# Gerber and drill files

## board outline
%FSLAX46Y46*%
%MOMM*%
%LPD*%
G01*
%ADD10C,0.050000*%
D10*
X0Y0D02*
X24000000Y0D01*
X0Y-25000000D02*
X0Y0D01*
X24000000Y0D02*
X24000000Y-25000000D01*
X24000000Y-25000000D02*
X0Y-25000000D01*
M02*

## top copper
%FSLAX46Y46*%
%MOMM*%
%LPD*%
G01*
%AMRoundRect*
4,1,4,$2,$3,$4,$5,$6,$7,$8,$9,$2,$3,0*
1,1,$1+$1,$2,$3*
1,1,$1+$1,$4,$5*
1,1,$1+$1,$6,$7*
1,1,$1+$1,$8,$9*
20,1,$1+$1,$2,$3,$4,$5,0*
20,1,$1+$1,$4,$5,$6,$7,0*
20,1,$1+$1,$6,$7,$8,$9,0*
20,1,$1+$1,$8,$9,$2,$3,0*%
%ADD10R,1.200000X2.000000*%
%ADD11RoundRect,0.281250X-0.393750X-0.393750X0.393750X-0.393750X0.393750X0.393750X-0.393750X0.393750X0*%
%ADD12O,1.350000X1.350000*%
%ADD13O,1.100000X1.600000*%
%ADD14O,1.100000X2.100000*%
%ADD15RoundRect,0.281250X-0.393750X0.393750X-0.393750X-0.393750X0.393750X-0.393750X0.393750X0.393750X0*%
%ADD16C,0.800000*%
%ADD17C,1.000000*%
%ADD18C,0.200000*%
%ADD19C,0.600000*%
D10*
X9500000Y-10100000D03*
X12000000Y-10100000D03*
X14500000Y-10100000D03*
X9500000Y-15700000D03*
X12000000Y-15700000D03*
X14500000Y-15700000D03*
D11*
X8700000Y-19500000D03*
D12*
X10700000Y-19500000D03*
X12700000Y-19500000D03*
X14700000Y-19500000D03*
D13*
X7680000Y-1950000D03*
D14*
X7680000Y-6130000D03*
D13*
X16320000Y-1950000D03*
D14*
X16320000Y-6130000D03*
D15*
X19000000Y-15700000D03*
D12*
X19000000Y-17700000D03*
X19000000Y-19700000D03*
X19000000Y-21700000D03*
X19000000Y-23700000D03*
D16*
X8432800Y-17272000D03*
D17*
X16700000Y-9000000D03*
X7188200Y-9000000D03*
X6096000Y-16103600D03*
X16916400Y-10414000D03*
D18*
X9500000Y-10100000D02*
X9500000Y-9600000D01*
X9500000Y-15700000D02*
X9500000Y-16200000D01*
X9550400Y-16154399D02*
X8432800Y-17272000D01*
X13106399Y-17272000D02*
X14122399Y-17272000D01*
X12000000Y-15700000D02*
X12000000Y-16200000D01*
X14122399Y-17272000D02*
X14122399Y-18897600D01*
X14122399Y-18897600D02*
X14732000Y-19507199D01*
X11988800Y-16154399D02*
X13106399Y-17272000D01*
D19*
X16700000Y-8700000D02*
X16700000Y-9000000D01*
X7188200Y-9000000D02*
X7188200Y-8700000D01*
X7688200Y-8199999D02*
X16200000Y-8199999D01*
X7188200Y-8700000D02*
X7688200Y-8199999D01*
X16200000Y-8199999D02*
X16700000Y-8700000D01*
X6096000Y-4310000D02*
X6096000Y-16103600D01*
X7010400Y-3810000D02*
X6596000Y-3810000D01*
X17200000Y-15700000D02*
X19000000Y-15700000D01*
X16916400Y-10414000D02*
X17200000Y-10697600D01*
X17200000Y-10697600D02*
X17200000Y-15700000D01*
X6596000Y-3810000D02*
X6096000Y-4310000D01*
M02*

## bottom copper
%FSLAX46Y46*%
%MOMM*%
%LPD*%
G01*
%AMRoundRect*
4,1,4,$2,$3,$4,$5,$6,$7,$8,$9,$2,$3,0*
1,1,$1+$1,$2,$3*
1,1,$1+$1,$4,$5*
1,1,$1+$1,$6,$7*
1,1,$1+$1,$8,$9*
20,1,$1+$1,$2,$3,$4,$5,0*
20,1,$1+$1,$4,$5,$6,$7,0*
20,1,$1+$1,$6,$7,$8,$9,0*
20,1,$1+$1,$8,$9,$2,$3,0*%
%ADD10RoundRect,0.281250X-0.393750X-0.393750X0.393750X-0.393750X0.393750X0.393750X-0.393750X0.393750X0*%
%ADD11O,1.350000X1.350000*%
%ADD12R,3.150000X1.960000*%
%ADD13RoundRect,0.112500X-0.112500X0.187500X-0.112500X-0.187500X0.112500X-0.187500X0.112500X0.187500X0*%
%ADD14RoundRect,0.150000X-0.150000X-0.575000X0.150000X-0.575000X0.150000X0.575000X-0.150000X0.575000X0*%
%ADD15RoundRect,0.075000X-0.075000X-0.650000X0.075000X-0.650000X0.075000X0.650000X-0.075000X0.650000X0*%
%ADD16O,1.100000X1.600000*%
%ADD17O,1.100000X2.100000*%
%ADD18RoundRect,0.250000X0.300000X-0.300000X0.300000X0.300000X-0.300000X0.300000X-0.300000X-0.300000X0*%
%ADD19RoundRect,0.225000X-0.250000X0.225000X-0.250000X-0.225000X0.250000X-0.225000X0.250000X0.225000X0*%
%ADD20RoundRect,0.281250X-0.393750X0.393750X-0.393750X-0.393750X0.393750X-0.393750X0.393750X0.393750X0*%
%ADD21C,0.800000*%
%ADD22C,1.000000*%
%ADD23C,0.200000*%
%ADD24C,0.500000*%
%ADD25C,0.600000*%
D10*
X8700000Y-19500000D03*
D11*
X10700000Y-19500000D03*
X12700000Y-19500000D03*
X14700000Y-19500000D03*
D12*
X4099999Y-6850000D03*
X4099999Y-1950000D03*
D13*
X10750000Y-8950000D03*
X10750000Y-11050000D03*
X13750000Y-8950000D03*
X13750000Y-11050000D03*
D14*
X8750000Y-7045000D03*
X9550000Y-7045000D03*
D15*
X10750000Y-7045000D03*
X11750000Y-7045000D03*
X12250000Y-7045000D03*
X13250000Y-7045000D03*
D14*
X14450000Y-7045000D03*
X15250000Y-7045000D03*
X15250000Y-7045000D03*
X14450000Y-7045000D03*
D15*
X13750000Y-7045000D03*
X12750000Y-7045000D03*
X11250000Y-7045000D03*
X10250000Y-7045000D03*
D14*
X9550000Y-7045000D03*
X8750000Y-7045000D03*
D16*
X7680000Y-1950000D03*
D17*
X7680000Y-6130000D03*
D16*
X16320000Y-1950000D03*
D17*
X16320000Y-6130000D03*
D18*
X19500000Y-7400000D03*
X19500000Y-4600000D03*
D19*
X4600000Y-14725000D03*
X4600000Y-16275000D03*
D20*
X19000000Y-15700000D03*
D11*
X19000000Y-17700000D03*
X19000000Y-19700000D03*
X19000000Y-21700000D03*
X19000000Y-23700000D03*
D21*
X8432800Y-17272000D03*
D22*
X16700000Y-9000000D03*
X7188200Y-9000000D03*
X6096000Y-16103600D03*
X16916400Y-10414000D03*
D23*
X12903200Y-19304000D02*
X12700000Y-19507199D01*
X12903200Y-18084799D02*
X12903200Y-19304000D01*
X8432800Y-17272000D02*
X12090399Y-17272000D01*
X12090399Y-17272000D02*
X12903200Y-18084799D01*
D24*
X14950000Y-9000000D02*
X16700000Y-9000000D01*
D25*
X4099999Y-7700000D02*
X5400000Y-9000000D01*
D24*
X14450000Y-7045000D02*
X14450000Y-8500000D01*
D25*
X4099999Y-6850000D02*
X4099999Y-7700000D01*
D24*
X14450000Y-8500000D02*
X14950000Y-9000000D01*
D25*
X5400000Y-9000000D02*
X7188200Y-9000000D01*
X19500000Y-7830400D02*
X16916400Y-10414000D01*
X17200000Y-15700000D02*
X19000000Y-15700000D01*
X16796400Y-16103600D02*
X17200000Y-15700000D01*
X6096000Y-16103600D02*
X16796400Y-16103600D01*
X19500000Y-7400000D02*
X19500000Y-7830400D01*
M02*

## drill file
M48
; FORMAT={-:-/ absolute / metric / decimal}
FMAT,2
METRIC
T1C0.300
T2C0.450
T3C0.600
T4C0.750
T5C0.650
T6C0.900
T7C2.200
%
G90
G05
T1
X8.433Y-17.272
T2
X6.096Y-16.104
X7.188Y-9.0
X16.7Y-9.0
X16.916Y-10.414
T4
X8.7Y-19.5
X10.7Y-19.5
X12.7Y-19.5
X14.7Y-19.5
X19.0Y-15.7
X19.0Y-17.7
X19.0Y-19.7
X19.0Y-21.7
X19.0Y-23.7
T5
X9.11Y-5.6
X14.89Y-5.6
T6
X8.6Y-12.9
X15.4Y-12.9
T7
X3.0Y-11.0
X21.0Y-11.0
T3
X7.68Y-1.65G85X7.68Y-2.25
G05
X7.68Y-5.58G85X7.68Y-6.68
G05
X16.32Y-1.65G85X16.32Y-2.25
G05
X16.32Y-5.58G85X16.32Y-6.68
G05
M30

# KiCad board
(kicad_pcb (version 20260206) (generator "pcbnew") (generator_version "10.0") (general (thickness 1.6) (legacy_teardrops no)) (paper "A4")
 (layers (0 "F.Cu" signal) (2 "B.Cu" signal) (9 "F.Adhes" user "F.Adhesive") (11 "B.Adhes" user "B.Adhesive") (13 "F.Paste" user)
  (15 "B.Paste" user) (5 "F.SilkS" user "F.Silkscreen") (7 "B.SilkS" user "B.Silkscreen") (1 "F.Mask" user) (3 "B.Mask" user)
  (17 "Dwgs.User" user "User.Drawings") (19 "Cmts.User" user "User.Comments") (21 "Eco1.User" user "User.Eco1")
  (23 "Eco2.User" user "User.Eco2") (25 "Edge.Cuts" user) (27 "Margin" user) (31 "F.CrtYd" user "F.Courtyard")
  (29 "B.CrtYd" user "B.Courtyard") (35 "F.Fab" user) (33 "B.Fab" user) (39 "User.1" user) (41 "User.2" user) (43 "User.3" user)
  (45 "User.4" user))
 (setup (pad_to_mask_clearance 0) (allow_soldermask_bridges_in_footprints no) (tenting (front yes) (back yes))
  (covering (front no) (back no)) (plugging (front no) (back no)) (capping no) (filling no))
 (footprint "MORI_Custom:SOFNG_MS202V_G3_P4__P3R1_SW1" (layer "F.Cu") (at 12 12.9)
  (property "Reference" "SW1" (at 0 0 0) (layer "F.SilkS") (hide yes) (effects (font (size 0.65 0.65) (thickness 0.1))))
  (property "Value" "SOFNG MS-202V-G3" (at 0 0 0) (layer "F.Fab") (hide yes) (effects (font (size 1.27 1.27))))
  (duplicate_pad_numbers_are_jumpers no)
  (pad "" np_thru_hole circle (at -3.4 0) (size 0.9 0.9) (drill 0.9) (layers "*.Cu" "*.Mask"))
  (pad "" np_thru_hole circle (at 3.4 0) (size 0.9 0.9) (drill 0.9) (layers "*.Cu" "*.Mask"))
  (pad "1" smd rect (at -2.5 -2.8) (size 1.2 2) (layers "F.Cu" "F.Mask" "F.Paste") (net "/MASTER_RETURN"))
  (pad "2" smd rect (at 0 -2.8) (size 1.2 2) (layers "F.Cu" "F.Mask" "F.Paste") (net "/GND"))
  (pad "3" smd rect (at 2.5 -2.8) (size 1.2 2) (layers "F.Cu" "F.Mask" "F.Paste") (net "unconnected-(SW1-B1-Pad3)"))
  (pad "4" smd rect (at -2.5 2.8) (size 1.2 2) (layers "F.Cu" "F.Mask" "F.Paste") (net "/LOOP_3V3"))
  (pad "5" smd rect (at 0 2.8) (size 1.2 2) (layers "F.Cu" "F.Mask" "F.Paste") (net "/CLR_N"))
  (pad "6" smd rect (at 2.5 2.8) (size 1.2 2) (layers "F.Cu" "F.Mask" "F.Paste") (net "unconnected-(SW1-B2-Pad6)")))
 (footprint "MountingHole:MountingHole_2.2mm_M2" (layer "F.Cu") (at 3 11)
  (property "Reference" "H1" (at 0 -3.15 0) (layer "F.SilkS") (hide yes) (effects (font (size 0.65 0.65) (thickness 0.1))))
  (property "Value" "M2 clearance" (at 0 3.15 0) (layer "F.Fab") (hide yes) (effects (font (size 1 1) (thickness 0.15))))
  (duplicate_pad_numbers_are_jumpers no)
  (pad "" np_thru_hole circle (at 0 0) (size 2.2 2.2) (drill 2.2) (layers "*.Cu" "*.Mask")))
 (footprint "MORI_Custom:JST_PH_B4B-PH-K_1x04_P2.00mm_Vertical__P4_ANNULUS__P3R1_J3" (layer "F.Cu") (at 8.7 19.5)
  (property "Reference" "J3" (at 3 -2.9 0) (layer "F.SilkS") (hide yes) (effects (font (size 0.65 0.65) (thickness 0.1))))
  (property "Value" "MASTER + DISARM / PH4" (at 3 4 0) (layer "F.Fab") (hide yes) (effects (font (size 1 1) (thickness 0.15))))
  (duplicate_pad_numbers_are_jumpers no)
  (pad "1" thru_hole roundrect (at 0 0) (size 1.35 1.35) (drill 0.75) (layers "*.Cu" "*.Mask") (remove_unused_layers no)
   (roundrect_rratio 0.208333) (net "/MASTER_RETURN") (thermal_bridge_width 0.299999) (thermal_bridge_angle 45) (thermal_gap 0.254))
  (pad "2" thru_hole oval (at 2 0) (size 1.35 1.35) (drill 0.75) (layers "*.Cu" "*.Mask") (remove_unused_layers no) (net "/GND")
   (thermal_bridge_width 0.299999) (thermal_bridge_angle 45) (thermal_gap 0.254))
  (pad "3" thru_hole oval (at 4 0) (size 1.35 1.35) (drill 0.75) (layers "*.Cu" "*.Mask") (remove_unused_layers no) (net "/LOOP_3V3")
   (thermal_bridge_width 0.299999) (thermal_bridge_angle 45) (thermal_gap 0.254))
  (pad "4" thru_hole oval (at 6 0) (size 1.35 1.35) (drill 0.75) (layers "*.Cu" "*.Mask") (remove_unused_layers no) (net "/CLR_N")
   (thermal_bridge_width 0.299999) (thermal_bridge_angle 45) (thermal_gap 0.254)))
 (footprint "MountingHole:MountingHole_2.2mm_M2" (layer "F.Cu") (at 21 11)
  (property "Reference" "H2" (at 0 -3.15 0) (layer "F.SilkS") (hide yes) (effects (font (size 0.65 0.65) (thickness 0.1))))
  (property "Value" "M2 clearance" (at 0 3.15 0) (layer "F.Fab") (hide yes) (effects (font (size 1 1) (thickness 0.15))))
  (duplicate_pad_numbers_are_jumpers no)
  (pad "" np_thru_hole circle (at 0 0) (size 2.2 2.2) (drill 2.2) (layers "*.Cu" "*.Mask")))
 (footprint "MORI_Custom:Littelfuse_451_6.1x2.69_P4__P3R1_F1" (layer "B.Cu") (at 4.099999 4.4 90)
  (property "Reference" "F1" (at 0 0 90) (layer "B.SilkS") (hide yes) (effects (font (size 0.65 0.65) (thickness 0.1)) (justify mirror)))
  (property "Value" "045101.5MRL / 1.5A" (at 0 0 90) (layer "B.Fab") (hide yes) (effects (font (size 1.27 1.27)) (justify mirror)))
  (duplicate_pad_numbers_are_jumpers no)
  (pad "1" smd rect (at -2.45 0 90) (size 1.96 3.15) (layers "B.Cu" "B.Mask" "B.Paste") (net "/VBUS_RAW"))
  (pad "2" smd rect (at 2.45 0 90) (size 1.96 3.15) (layers "B.Cu" "B.Mask" "B.Paste") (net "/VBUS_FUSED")))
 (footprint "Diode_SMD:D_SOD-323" (layer "B.Cu") (at 10.75 10 -90)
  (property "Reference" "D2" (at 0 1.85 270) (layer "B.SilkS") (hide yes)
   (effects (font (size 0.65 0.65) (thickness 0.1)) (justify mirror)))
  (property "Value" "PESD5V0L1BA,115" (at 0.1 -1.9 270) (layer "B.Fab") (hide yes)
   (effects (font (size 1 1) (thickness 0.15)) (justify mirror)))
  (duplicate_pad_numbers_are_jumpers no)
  (pad "1" smd roundrect (at -1.05 0 270) (size 0.6 0.45) (layers "B.Cu" "B.Mask" "B.Paste") (roundrect_rratio 0.25) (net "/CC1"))
  (pad "2" smd roundrect (at 1.05 0 270) (size 0.6 0.45) (layers "B.Cu" "B.Mask" "B.Paste") (roundrect_rratio 0.25) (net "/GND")))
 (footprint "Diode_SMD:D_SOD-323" (layer "B.Cu") (at 13.75 10 -90)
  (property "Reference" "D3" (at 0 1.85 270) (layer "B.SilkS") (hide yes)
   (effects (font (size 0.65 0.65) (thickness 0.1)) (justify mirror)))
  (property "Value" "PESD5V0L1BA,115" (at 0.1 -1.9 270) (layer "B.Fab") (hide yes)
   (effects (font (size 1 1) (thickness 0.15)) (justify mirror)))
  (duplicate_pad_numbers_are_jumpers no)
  (pad "1" smd roundrect (at -1.05 0 270) (size 0.6 0.45) (layers "B.Cu" "B.Mask" "B.Paste") (roundrect_rratio 0.25) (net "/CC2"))
  (pad "2" smd roundrect (at 1.05 0 270) (size 0.6 0.45) (layers "B.Cu" "B.Mask" "B.Paste") (roundrect_rratio 0.25) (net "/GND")))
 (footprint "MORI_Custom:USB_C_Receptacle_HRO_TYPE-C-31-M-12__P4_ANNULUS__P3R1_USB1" (layer "B.Cu") (at 12 3)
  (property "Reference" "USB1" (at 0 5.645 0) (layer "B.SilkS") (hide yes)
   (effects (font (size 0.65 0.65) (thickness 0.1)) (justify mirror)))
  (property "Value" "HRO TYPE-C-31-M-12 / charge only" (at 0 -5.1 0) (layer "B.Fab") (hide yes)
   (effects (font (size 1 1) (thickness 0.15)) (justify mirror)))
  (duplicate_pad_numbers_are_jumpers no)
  (pad "" np_thru_hole circle (at -2.89 2.6) (size 0.65 0.65) (drill 0.65) (layers "*.Cu" "*.Mask"))
  (pad "" np_thru_hole circle (at 2.89 2.6) (size 0.65 0.65) (drill 0.65) (layers "*.Cu" "*.Mask"))
  (pad "A1" smd roundrect (at -3.25 4.045) (size 0.6 1.45) (layers "B.Cu" "B.Mask" "B.Paste") (roundrect_rratio 0.25) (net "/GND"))
  (pad "A4" smd roundrect (at -2.45 4.045) (size 0.6 1.45) (layers "B.Cu" "B.Mask" "B.Paste") (roundrect_rratio 0.25) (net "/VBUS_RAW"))
  (pad "A5" smd roundrect (at -1.25 4.045) (size 0.3 1.45) (layers "B.Cu" "B.Mask" "B.Paste") (roundrect_rratio 0.25) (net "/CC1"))
  (pad "A6" smd roundrect (at -0.25 4.045) (size 0.3 1.45) (layers "B.Cu" "B.Mask" "B.Paste") (roundrect_rratio 0.25)
   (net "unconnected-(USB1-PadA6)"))
  (pad "A7" smd roundrect (at 0.25 4.045) (size 0.3 1.45) (layers "B.Cu" "B.Mask" "B.Paste") (roundrect_rratio 0.25)
   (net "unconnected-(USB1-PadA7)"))
  (pad "A8" smd roundrect (at 1.25 4.045) (size 0.3 1.45) (layers "B.Cu" "B.Mask" "B.Paste") (roundrect_rratio 0.25)
   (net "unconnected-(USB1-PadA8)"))
  (pad "A9" smd roundrect (at 2.45 4.045) (size 0.6 1.45) (layers "B.Cu" "B.Mask" "B.Paste") (roundrect_rratio 0.25) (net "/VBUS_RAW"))
  (pad "A12" smd roundrect (at 3.25 4.045) (size 0.6 1.45) (layers "B.Cu" "B.Mask" "B.Paste") (roundrect_rratio 0.25) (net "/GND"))
  (pad "B1" smd roundrect (at 3.25 4.045) (size 0.6 1.45) (layers "B.Cu" "B.Mask" "B.Paste") (roundrect_rratio 0.25) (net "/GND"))
  (pad "B4" smd roundrect (at 2.45 4.045) (size 0.6 1.45) (layers "B.Cu" "B.Mask" "B.Paste") (roundrect_rratio 0.25) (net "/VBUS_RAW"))
  (pad "B5" smd roundrect (at 1.75 4.045) (size 0.3 1.45) (layers "B.Cu" "B.Mask" "B.Paste") (roundrect_rratio 0.25) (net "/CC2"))
  (pad "B6" smd roundrect (at 0.75 4.045) (size 0.3 1.45) (layers "B.Cu" "B.Mask" "B.Paste") (roundrect_rratio 0.25)
   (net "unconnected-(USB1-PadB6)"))
  (pad "B7" smd roundrect (at -0.75 4.045) (size 0.3 1.45) (layers "B.Cu" "B.Mask" "B.Paste") (roundrect_rratio 0.25)
   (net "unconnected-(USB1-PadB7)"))
  (pad "B8" smd roundrect (at -1.75 4.045) (size 0.3 1.45) (layers "B.Cu" "B.Mask" "B.Paste") (roundrect_rratio 0.25)
   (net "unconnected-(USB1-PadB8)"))
  (pad "B9" smd roundrect (at -2.45 4.045) (size 0.6 1.45) (layers "B.Cu" "B.Mask" "B.Paste") (roundrect_rratio 0.25) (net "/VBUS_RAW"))
  (pad "B12" smd roundrect (at -3.25 4.045) (size 0.6 1.45) (layers "B.Cu" "B.Mask" "B.Paste") (roundrect_rratio 0.25) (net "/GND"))
  (pad "SH" thru_hole oval (at -4.32 -1.05) (size 1.1 1.6) (drill oval 0.6 1.2) (layers "*.Cu" "*.Mask") (remove_unused_layers no)
   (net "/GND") (thermal_bridge_width 0.299999) (thermal_bridge_angle 45) (thermal_gap 0.254))
  (pad "SH" thru_hole oval (at -4.32 3.13) (size 1.1 2.1) (drill oval 0.6 1.7) (layers "*.Cu" "*.Mask") (remove_unused_layers no)
   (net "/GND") (thermal_bridge_width 0.299999) (thermal_bridge_angle 45) (thermal_gap 0.254))
  (pad "SH" thru_hole oval (at 4.32 -1.05) (size 1.1 1.6) (drill oval 0.6 1.2) (layers "*.Cu" "*.Mask") (remove_unused_layers no)
   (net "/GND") (thermal_bridge_width 0.299999) (thermal_bridge_angle 45) (thermal_gap 0.254))
  (pad "SH" thru_hole oval (at 4.32 3.13) (size 1.1 2.1) (drill oval 0.6 1.7) (layers "*.Cu" "*.Mask") (remove_unused_layers no)
   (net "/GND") (thermal_bridge_width 0.299999) (thermal_bridge_angle 45) (thermal_gap 0.254)))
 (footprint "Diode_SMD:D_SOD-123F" (layer "B.Cu") (at 19.5 6 90)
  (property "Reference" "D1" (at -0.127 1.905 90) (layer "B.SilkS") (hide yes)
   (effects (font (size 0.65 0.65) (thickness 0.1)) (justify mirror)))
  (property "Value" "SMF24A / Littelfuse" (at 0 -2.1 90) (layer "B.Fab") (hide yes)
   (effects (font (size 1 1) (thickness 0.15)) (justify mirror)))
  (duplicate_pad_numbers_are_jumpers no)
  (pad "1" smd roundrect (at -1.4 0 90) (size 1.1 1.1) (layers "B.Cu" "B.Mask" "B.Paste") (roundrect_rratio 0.2272727273)
   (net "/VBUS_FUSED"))
  (pad "2" smd roundrect (at 1.4 0 90) (size 1.1 1.1) (layers "B.Cu" "B.Mask" "B.Paste") (roundrect_rratio 0.2272727273) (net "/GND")))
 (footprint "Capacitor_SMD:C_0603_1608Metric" (layer "B.Cu") (at 4.6 15.5 -90)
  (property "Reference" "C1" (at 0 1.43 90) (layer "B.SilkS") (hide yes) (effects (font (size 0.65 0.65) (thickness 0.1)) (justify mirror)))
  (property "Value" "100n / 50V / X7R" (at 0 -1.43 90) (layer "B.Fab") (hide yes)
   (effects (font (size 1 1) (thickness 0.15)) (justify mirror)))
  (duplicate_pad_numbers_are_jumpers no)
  (pad "1" smd roundrect (at -0.775 0 270) (size 0.9 0.95) (layers "B.Cu" "B.Mask" "B.Paste") (roundrect_rratio 0.25) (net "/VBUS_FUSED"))
  (pad "2" smd roundrect (at 0.775 0 270) (size 0.9 0.95) (layers "B.Cu" "B.Mask" "B.Paste") (roundrect_rratio 0.25) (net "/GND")))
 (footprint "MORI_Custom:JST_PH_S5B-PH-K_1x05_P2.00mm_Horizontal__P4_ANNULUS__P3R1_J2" (layer "B.Cu") (at 19 15.7 -90)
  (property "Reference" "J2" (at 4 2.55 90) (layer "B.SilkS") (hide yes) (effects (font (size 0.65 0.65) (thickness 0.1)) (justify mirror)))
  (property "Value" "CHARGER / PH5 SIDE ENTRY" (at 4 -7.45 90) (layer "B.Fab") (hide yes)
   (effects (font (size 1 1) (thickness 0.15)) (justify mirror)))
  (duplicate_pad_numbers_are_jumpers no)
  (pad "1" thru_hole roundrect (at 0 0 270) (size 1.35 1.35) (drill 0.75) (layers "*.Cu" "*.Mask") (remove_unused_layers no)
   (roundrect_rratio 0.208333) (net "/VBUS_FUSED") (thermal_bridge_width 0.299999) (thermal_bridge_angle 45) (thermal_gap 0.254))
  (pad "2" thru_hole oval (at 2 0 270) (size 1.35 1.35) (drill 0.75) (layers "*.Cu" "*.Mask") (remove_unused_layers no) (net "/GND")
   (thermal_bridge_width 0.299999) (thermal_bridge_angle 45) (thermal_gap 0.254))
  (pad "3" thru_hole oval (at 4 0 270) (size 1.35 1.35) (drill 0.75) (layers "*.Cu" "*.Mask") (remove_unused_layers no) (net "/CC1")
   (thermal_bridge_width 0.299999) (thermal_bridge_angle 45) (thermal_gap 0.254))
  (pad "4" thru_hole oval (at 6 0 270) (size 1.35 1.35) (drill 0.75) (layers "*.Cu" "*.Mask") (remove_unused_layers no) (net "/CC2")
   (thermal_bridge_width 0.299999) (thermal_bridge_angle 45) (thermal_gap 0.254))
  (pad "5" thru_hole oval (at 8 0 270) (size 1.35 1.35) (drill 0.75) (layers "*.Cu" "*.Mask") (remove_unused_layers no) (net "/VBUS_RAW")
   (thermal_bridge_width 0.299999) (thermal_bridge_angle 45) (thermal_gap 0.254)))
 (gr_line (start 0 0) (end 24 0) (stroke (width 0.05) (type default)) (layer "Edge.Cuts"))
 (gr_line (start 0 25) (end 0 0) (stroke (width 0.05) (type default)) (layer "Edge.Cuts"))
 (gr_line (start 24 0) (end 24 25) (stroke (width 0.05) (type default)) (layer "Edge.Cuts"))
 (gr_line (start 24 25) (end 0 25) (stroke (width 0.05) (type default)) (layer "Edge.Cuts"))
 (segment (start 9.5 10.1) (end 9.5 9.6) (width 0.2) (layer "F.Cu") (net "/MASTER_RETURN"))
 (segment (start 9.5 15.7) (end 9.5 16.2) (width 0.2) (layer "F.Cu") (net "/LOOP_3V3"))
 (segment (start 9.5504 16.154399) (end 8.4328 17.272) (width 0.2) (layer "F.Cu") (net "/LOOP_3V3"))
 (via (at 8.4328 17.272) (size 0.8) (drill 0.3) (layers "F.Cu" "B.Cu") (tenting (front no) (back none)) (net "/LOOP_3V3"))
 (segment (start 12.9032 19.304) (end 12.7 19.507199) (width 0.2) (layer "B.Cu") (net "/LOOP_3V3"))
 (segment (start 12.9032 18.084799) (end 12.9032 19.304) (width 0.2) (layer "B.Cu") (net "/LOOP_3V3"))
 (segment (start 8.4328 17.272) (end 12.090399 17.272) (width 0.2) (layer "B.Cu") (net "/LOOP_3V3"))
 (segment (start 12.090399 17.272) (end 12.9032 18.084799) (width 0.2) (layer "B.Cu") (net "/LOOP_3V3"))
 (segment (start 13.106399 17.272) (end 14.122399 17.272) (width 0.2) (layer "F.Cu") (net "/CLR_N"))
 (segment (start 12 15.7) (end 12 16.2) (width 0.2) (layer "F.Cu") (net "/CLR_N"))
 (segment (start 14.122399 17.272) (end 14.122399 18.8976) (width 0.2) (layer "F.Cu") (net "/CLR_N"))
 (segment (start 14.122399 18.8976) (end 14.732 19.507199) (width 0.2) (layer "F.Cu") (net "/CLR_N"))
 (segment (start 11.9888 16.154399) (end 13.106399 17.272) (width 0.2) (layer "F.Cu") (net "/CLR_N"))
 (segment (start 16.7 8.7) (end 16.7 9) (width 0.6) (layer "F.Cu") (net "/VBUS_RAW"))
 (segment (start 7.1882 9) (end 7.1882 8.7) (width 0.6) (layer "F.Cu") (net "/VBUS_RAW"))
 (segment (start 7.6882 8.199999) (end 16.2 8.199999) (width 0.6) (layer "F.Cu") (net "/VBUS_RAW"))
 (segment (start 7.1882 8.7) (end 7.6882 8.199999) (width 0.6) (layer "F.Cu") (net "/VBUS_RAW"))
 (segment (start 16.2 8.199999) (end 16.7 8.7) (width 0.6) (layer "F.Cu") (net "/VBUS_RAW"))
 (via (at 16.7 9) (size 1) (drill 0.45) (layers "F.Cu" "B.Cu") (tenting (front no) (back none)) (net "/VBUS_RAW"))
 (via (at 7.1882 9) (size 1) (drill 0.45) (layers "F.Cu" "B.Cu") (tenting (front no) (back none)) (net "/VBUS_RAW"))
 (segment (start 14.95 9) (end 16.7 9) (width 0.5) (layer "B.Cu") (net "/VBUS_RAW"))
 (segment (start 4.099999 7.7) (end 5.4 9) (width 0.6) (layer "B.Cu") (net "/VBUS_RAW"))
 (segment (start 14.45 7.045) (end 14.45 8.5) (width 0.5) (layer "B.Cu") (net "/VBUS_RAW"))
 (segment (start 4.099999 6.85) (end 4.099999 7.7) (width 0.6) (layer "B.Cu") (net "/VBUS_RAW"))
 (segment (start 14.45 8.5) (end 14.95 9) (width 0.5) (layer "B.Cu") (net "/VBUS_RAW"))
 (segment (start 5.4 9) (end 7.1882 9) (width 0.6) (layer "B.Cu") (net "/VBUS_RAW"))
 (segment (start 6.096 4.31) (end 6.096 16.1036) (width 0.6) (layer "F.Cu") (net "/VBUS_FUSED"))
 (segment (start 7.0104 3.81) (end 6.596 3.81) (width 0.6) (layer "F.Cu") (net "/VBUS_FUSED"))
 (segment (start 17.2 15.7) (end 19 15.7) (width 0.6) (layer "F.Cu") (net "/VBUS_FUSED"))
 (segment (start 16.9164 10.414) (end 17.2 10.6976) (width 0.6) (layer "F.Cu") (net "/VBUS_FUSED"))
 (segment (start 17.2 10.6976) (end 17.2 15.7) (width 0.6) (layer "F.Cu") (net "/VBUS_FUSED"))
 (segment (start 6.596 3.81) (end 6.096 4.31) (width 0.6) (layer "F.Cu") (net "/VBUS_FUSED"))
 (via (at 6.096 16.1036) (size 1) (drill 0.45) (layers "F.Cu" "B.Cu") (tenting (front no) (back none)) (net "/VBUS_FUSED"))
 (via (at 16.9164 10.414) (size 1) (drill 0.45) (layers "F.Cu" "B.Cu") (tenting (front no) (back none)) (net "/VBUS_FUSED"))
 (segment (start 19.5 7.8304) (end 16.9164 10.414) (width 0.6) (layer "B.Cu") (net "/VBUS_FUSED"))
 (segment (start 17.2 15.7) (end 19 15.7) (width 0.6) (layer "B.Cu") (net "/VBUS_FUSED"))
 (segment (start 16.7964 16.1036) (end 17.2 15.7) (width 0.6) (layer "B.Cu") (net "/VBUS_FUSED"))
 (segment (start 6.096 16.1036) (end 16.7964 16.1036) (width 0.6) (layer "B.Cu") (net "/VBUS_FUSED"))
 (segment (start 19.5 7.4) (end 19.5 7.8304) (width 0.6) (layer "B.Cu") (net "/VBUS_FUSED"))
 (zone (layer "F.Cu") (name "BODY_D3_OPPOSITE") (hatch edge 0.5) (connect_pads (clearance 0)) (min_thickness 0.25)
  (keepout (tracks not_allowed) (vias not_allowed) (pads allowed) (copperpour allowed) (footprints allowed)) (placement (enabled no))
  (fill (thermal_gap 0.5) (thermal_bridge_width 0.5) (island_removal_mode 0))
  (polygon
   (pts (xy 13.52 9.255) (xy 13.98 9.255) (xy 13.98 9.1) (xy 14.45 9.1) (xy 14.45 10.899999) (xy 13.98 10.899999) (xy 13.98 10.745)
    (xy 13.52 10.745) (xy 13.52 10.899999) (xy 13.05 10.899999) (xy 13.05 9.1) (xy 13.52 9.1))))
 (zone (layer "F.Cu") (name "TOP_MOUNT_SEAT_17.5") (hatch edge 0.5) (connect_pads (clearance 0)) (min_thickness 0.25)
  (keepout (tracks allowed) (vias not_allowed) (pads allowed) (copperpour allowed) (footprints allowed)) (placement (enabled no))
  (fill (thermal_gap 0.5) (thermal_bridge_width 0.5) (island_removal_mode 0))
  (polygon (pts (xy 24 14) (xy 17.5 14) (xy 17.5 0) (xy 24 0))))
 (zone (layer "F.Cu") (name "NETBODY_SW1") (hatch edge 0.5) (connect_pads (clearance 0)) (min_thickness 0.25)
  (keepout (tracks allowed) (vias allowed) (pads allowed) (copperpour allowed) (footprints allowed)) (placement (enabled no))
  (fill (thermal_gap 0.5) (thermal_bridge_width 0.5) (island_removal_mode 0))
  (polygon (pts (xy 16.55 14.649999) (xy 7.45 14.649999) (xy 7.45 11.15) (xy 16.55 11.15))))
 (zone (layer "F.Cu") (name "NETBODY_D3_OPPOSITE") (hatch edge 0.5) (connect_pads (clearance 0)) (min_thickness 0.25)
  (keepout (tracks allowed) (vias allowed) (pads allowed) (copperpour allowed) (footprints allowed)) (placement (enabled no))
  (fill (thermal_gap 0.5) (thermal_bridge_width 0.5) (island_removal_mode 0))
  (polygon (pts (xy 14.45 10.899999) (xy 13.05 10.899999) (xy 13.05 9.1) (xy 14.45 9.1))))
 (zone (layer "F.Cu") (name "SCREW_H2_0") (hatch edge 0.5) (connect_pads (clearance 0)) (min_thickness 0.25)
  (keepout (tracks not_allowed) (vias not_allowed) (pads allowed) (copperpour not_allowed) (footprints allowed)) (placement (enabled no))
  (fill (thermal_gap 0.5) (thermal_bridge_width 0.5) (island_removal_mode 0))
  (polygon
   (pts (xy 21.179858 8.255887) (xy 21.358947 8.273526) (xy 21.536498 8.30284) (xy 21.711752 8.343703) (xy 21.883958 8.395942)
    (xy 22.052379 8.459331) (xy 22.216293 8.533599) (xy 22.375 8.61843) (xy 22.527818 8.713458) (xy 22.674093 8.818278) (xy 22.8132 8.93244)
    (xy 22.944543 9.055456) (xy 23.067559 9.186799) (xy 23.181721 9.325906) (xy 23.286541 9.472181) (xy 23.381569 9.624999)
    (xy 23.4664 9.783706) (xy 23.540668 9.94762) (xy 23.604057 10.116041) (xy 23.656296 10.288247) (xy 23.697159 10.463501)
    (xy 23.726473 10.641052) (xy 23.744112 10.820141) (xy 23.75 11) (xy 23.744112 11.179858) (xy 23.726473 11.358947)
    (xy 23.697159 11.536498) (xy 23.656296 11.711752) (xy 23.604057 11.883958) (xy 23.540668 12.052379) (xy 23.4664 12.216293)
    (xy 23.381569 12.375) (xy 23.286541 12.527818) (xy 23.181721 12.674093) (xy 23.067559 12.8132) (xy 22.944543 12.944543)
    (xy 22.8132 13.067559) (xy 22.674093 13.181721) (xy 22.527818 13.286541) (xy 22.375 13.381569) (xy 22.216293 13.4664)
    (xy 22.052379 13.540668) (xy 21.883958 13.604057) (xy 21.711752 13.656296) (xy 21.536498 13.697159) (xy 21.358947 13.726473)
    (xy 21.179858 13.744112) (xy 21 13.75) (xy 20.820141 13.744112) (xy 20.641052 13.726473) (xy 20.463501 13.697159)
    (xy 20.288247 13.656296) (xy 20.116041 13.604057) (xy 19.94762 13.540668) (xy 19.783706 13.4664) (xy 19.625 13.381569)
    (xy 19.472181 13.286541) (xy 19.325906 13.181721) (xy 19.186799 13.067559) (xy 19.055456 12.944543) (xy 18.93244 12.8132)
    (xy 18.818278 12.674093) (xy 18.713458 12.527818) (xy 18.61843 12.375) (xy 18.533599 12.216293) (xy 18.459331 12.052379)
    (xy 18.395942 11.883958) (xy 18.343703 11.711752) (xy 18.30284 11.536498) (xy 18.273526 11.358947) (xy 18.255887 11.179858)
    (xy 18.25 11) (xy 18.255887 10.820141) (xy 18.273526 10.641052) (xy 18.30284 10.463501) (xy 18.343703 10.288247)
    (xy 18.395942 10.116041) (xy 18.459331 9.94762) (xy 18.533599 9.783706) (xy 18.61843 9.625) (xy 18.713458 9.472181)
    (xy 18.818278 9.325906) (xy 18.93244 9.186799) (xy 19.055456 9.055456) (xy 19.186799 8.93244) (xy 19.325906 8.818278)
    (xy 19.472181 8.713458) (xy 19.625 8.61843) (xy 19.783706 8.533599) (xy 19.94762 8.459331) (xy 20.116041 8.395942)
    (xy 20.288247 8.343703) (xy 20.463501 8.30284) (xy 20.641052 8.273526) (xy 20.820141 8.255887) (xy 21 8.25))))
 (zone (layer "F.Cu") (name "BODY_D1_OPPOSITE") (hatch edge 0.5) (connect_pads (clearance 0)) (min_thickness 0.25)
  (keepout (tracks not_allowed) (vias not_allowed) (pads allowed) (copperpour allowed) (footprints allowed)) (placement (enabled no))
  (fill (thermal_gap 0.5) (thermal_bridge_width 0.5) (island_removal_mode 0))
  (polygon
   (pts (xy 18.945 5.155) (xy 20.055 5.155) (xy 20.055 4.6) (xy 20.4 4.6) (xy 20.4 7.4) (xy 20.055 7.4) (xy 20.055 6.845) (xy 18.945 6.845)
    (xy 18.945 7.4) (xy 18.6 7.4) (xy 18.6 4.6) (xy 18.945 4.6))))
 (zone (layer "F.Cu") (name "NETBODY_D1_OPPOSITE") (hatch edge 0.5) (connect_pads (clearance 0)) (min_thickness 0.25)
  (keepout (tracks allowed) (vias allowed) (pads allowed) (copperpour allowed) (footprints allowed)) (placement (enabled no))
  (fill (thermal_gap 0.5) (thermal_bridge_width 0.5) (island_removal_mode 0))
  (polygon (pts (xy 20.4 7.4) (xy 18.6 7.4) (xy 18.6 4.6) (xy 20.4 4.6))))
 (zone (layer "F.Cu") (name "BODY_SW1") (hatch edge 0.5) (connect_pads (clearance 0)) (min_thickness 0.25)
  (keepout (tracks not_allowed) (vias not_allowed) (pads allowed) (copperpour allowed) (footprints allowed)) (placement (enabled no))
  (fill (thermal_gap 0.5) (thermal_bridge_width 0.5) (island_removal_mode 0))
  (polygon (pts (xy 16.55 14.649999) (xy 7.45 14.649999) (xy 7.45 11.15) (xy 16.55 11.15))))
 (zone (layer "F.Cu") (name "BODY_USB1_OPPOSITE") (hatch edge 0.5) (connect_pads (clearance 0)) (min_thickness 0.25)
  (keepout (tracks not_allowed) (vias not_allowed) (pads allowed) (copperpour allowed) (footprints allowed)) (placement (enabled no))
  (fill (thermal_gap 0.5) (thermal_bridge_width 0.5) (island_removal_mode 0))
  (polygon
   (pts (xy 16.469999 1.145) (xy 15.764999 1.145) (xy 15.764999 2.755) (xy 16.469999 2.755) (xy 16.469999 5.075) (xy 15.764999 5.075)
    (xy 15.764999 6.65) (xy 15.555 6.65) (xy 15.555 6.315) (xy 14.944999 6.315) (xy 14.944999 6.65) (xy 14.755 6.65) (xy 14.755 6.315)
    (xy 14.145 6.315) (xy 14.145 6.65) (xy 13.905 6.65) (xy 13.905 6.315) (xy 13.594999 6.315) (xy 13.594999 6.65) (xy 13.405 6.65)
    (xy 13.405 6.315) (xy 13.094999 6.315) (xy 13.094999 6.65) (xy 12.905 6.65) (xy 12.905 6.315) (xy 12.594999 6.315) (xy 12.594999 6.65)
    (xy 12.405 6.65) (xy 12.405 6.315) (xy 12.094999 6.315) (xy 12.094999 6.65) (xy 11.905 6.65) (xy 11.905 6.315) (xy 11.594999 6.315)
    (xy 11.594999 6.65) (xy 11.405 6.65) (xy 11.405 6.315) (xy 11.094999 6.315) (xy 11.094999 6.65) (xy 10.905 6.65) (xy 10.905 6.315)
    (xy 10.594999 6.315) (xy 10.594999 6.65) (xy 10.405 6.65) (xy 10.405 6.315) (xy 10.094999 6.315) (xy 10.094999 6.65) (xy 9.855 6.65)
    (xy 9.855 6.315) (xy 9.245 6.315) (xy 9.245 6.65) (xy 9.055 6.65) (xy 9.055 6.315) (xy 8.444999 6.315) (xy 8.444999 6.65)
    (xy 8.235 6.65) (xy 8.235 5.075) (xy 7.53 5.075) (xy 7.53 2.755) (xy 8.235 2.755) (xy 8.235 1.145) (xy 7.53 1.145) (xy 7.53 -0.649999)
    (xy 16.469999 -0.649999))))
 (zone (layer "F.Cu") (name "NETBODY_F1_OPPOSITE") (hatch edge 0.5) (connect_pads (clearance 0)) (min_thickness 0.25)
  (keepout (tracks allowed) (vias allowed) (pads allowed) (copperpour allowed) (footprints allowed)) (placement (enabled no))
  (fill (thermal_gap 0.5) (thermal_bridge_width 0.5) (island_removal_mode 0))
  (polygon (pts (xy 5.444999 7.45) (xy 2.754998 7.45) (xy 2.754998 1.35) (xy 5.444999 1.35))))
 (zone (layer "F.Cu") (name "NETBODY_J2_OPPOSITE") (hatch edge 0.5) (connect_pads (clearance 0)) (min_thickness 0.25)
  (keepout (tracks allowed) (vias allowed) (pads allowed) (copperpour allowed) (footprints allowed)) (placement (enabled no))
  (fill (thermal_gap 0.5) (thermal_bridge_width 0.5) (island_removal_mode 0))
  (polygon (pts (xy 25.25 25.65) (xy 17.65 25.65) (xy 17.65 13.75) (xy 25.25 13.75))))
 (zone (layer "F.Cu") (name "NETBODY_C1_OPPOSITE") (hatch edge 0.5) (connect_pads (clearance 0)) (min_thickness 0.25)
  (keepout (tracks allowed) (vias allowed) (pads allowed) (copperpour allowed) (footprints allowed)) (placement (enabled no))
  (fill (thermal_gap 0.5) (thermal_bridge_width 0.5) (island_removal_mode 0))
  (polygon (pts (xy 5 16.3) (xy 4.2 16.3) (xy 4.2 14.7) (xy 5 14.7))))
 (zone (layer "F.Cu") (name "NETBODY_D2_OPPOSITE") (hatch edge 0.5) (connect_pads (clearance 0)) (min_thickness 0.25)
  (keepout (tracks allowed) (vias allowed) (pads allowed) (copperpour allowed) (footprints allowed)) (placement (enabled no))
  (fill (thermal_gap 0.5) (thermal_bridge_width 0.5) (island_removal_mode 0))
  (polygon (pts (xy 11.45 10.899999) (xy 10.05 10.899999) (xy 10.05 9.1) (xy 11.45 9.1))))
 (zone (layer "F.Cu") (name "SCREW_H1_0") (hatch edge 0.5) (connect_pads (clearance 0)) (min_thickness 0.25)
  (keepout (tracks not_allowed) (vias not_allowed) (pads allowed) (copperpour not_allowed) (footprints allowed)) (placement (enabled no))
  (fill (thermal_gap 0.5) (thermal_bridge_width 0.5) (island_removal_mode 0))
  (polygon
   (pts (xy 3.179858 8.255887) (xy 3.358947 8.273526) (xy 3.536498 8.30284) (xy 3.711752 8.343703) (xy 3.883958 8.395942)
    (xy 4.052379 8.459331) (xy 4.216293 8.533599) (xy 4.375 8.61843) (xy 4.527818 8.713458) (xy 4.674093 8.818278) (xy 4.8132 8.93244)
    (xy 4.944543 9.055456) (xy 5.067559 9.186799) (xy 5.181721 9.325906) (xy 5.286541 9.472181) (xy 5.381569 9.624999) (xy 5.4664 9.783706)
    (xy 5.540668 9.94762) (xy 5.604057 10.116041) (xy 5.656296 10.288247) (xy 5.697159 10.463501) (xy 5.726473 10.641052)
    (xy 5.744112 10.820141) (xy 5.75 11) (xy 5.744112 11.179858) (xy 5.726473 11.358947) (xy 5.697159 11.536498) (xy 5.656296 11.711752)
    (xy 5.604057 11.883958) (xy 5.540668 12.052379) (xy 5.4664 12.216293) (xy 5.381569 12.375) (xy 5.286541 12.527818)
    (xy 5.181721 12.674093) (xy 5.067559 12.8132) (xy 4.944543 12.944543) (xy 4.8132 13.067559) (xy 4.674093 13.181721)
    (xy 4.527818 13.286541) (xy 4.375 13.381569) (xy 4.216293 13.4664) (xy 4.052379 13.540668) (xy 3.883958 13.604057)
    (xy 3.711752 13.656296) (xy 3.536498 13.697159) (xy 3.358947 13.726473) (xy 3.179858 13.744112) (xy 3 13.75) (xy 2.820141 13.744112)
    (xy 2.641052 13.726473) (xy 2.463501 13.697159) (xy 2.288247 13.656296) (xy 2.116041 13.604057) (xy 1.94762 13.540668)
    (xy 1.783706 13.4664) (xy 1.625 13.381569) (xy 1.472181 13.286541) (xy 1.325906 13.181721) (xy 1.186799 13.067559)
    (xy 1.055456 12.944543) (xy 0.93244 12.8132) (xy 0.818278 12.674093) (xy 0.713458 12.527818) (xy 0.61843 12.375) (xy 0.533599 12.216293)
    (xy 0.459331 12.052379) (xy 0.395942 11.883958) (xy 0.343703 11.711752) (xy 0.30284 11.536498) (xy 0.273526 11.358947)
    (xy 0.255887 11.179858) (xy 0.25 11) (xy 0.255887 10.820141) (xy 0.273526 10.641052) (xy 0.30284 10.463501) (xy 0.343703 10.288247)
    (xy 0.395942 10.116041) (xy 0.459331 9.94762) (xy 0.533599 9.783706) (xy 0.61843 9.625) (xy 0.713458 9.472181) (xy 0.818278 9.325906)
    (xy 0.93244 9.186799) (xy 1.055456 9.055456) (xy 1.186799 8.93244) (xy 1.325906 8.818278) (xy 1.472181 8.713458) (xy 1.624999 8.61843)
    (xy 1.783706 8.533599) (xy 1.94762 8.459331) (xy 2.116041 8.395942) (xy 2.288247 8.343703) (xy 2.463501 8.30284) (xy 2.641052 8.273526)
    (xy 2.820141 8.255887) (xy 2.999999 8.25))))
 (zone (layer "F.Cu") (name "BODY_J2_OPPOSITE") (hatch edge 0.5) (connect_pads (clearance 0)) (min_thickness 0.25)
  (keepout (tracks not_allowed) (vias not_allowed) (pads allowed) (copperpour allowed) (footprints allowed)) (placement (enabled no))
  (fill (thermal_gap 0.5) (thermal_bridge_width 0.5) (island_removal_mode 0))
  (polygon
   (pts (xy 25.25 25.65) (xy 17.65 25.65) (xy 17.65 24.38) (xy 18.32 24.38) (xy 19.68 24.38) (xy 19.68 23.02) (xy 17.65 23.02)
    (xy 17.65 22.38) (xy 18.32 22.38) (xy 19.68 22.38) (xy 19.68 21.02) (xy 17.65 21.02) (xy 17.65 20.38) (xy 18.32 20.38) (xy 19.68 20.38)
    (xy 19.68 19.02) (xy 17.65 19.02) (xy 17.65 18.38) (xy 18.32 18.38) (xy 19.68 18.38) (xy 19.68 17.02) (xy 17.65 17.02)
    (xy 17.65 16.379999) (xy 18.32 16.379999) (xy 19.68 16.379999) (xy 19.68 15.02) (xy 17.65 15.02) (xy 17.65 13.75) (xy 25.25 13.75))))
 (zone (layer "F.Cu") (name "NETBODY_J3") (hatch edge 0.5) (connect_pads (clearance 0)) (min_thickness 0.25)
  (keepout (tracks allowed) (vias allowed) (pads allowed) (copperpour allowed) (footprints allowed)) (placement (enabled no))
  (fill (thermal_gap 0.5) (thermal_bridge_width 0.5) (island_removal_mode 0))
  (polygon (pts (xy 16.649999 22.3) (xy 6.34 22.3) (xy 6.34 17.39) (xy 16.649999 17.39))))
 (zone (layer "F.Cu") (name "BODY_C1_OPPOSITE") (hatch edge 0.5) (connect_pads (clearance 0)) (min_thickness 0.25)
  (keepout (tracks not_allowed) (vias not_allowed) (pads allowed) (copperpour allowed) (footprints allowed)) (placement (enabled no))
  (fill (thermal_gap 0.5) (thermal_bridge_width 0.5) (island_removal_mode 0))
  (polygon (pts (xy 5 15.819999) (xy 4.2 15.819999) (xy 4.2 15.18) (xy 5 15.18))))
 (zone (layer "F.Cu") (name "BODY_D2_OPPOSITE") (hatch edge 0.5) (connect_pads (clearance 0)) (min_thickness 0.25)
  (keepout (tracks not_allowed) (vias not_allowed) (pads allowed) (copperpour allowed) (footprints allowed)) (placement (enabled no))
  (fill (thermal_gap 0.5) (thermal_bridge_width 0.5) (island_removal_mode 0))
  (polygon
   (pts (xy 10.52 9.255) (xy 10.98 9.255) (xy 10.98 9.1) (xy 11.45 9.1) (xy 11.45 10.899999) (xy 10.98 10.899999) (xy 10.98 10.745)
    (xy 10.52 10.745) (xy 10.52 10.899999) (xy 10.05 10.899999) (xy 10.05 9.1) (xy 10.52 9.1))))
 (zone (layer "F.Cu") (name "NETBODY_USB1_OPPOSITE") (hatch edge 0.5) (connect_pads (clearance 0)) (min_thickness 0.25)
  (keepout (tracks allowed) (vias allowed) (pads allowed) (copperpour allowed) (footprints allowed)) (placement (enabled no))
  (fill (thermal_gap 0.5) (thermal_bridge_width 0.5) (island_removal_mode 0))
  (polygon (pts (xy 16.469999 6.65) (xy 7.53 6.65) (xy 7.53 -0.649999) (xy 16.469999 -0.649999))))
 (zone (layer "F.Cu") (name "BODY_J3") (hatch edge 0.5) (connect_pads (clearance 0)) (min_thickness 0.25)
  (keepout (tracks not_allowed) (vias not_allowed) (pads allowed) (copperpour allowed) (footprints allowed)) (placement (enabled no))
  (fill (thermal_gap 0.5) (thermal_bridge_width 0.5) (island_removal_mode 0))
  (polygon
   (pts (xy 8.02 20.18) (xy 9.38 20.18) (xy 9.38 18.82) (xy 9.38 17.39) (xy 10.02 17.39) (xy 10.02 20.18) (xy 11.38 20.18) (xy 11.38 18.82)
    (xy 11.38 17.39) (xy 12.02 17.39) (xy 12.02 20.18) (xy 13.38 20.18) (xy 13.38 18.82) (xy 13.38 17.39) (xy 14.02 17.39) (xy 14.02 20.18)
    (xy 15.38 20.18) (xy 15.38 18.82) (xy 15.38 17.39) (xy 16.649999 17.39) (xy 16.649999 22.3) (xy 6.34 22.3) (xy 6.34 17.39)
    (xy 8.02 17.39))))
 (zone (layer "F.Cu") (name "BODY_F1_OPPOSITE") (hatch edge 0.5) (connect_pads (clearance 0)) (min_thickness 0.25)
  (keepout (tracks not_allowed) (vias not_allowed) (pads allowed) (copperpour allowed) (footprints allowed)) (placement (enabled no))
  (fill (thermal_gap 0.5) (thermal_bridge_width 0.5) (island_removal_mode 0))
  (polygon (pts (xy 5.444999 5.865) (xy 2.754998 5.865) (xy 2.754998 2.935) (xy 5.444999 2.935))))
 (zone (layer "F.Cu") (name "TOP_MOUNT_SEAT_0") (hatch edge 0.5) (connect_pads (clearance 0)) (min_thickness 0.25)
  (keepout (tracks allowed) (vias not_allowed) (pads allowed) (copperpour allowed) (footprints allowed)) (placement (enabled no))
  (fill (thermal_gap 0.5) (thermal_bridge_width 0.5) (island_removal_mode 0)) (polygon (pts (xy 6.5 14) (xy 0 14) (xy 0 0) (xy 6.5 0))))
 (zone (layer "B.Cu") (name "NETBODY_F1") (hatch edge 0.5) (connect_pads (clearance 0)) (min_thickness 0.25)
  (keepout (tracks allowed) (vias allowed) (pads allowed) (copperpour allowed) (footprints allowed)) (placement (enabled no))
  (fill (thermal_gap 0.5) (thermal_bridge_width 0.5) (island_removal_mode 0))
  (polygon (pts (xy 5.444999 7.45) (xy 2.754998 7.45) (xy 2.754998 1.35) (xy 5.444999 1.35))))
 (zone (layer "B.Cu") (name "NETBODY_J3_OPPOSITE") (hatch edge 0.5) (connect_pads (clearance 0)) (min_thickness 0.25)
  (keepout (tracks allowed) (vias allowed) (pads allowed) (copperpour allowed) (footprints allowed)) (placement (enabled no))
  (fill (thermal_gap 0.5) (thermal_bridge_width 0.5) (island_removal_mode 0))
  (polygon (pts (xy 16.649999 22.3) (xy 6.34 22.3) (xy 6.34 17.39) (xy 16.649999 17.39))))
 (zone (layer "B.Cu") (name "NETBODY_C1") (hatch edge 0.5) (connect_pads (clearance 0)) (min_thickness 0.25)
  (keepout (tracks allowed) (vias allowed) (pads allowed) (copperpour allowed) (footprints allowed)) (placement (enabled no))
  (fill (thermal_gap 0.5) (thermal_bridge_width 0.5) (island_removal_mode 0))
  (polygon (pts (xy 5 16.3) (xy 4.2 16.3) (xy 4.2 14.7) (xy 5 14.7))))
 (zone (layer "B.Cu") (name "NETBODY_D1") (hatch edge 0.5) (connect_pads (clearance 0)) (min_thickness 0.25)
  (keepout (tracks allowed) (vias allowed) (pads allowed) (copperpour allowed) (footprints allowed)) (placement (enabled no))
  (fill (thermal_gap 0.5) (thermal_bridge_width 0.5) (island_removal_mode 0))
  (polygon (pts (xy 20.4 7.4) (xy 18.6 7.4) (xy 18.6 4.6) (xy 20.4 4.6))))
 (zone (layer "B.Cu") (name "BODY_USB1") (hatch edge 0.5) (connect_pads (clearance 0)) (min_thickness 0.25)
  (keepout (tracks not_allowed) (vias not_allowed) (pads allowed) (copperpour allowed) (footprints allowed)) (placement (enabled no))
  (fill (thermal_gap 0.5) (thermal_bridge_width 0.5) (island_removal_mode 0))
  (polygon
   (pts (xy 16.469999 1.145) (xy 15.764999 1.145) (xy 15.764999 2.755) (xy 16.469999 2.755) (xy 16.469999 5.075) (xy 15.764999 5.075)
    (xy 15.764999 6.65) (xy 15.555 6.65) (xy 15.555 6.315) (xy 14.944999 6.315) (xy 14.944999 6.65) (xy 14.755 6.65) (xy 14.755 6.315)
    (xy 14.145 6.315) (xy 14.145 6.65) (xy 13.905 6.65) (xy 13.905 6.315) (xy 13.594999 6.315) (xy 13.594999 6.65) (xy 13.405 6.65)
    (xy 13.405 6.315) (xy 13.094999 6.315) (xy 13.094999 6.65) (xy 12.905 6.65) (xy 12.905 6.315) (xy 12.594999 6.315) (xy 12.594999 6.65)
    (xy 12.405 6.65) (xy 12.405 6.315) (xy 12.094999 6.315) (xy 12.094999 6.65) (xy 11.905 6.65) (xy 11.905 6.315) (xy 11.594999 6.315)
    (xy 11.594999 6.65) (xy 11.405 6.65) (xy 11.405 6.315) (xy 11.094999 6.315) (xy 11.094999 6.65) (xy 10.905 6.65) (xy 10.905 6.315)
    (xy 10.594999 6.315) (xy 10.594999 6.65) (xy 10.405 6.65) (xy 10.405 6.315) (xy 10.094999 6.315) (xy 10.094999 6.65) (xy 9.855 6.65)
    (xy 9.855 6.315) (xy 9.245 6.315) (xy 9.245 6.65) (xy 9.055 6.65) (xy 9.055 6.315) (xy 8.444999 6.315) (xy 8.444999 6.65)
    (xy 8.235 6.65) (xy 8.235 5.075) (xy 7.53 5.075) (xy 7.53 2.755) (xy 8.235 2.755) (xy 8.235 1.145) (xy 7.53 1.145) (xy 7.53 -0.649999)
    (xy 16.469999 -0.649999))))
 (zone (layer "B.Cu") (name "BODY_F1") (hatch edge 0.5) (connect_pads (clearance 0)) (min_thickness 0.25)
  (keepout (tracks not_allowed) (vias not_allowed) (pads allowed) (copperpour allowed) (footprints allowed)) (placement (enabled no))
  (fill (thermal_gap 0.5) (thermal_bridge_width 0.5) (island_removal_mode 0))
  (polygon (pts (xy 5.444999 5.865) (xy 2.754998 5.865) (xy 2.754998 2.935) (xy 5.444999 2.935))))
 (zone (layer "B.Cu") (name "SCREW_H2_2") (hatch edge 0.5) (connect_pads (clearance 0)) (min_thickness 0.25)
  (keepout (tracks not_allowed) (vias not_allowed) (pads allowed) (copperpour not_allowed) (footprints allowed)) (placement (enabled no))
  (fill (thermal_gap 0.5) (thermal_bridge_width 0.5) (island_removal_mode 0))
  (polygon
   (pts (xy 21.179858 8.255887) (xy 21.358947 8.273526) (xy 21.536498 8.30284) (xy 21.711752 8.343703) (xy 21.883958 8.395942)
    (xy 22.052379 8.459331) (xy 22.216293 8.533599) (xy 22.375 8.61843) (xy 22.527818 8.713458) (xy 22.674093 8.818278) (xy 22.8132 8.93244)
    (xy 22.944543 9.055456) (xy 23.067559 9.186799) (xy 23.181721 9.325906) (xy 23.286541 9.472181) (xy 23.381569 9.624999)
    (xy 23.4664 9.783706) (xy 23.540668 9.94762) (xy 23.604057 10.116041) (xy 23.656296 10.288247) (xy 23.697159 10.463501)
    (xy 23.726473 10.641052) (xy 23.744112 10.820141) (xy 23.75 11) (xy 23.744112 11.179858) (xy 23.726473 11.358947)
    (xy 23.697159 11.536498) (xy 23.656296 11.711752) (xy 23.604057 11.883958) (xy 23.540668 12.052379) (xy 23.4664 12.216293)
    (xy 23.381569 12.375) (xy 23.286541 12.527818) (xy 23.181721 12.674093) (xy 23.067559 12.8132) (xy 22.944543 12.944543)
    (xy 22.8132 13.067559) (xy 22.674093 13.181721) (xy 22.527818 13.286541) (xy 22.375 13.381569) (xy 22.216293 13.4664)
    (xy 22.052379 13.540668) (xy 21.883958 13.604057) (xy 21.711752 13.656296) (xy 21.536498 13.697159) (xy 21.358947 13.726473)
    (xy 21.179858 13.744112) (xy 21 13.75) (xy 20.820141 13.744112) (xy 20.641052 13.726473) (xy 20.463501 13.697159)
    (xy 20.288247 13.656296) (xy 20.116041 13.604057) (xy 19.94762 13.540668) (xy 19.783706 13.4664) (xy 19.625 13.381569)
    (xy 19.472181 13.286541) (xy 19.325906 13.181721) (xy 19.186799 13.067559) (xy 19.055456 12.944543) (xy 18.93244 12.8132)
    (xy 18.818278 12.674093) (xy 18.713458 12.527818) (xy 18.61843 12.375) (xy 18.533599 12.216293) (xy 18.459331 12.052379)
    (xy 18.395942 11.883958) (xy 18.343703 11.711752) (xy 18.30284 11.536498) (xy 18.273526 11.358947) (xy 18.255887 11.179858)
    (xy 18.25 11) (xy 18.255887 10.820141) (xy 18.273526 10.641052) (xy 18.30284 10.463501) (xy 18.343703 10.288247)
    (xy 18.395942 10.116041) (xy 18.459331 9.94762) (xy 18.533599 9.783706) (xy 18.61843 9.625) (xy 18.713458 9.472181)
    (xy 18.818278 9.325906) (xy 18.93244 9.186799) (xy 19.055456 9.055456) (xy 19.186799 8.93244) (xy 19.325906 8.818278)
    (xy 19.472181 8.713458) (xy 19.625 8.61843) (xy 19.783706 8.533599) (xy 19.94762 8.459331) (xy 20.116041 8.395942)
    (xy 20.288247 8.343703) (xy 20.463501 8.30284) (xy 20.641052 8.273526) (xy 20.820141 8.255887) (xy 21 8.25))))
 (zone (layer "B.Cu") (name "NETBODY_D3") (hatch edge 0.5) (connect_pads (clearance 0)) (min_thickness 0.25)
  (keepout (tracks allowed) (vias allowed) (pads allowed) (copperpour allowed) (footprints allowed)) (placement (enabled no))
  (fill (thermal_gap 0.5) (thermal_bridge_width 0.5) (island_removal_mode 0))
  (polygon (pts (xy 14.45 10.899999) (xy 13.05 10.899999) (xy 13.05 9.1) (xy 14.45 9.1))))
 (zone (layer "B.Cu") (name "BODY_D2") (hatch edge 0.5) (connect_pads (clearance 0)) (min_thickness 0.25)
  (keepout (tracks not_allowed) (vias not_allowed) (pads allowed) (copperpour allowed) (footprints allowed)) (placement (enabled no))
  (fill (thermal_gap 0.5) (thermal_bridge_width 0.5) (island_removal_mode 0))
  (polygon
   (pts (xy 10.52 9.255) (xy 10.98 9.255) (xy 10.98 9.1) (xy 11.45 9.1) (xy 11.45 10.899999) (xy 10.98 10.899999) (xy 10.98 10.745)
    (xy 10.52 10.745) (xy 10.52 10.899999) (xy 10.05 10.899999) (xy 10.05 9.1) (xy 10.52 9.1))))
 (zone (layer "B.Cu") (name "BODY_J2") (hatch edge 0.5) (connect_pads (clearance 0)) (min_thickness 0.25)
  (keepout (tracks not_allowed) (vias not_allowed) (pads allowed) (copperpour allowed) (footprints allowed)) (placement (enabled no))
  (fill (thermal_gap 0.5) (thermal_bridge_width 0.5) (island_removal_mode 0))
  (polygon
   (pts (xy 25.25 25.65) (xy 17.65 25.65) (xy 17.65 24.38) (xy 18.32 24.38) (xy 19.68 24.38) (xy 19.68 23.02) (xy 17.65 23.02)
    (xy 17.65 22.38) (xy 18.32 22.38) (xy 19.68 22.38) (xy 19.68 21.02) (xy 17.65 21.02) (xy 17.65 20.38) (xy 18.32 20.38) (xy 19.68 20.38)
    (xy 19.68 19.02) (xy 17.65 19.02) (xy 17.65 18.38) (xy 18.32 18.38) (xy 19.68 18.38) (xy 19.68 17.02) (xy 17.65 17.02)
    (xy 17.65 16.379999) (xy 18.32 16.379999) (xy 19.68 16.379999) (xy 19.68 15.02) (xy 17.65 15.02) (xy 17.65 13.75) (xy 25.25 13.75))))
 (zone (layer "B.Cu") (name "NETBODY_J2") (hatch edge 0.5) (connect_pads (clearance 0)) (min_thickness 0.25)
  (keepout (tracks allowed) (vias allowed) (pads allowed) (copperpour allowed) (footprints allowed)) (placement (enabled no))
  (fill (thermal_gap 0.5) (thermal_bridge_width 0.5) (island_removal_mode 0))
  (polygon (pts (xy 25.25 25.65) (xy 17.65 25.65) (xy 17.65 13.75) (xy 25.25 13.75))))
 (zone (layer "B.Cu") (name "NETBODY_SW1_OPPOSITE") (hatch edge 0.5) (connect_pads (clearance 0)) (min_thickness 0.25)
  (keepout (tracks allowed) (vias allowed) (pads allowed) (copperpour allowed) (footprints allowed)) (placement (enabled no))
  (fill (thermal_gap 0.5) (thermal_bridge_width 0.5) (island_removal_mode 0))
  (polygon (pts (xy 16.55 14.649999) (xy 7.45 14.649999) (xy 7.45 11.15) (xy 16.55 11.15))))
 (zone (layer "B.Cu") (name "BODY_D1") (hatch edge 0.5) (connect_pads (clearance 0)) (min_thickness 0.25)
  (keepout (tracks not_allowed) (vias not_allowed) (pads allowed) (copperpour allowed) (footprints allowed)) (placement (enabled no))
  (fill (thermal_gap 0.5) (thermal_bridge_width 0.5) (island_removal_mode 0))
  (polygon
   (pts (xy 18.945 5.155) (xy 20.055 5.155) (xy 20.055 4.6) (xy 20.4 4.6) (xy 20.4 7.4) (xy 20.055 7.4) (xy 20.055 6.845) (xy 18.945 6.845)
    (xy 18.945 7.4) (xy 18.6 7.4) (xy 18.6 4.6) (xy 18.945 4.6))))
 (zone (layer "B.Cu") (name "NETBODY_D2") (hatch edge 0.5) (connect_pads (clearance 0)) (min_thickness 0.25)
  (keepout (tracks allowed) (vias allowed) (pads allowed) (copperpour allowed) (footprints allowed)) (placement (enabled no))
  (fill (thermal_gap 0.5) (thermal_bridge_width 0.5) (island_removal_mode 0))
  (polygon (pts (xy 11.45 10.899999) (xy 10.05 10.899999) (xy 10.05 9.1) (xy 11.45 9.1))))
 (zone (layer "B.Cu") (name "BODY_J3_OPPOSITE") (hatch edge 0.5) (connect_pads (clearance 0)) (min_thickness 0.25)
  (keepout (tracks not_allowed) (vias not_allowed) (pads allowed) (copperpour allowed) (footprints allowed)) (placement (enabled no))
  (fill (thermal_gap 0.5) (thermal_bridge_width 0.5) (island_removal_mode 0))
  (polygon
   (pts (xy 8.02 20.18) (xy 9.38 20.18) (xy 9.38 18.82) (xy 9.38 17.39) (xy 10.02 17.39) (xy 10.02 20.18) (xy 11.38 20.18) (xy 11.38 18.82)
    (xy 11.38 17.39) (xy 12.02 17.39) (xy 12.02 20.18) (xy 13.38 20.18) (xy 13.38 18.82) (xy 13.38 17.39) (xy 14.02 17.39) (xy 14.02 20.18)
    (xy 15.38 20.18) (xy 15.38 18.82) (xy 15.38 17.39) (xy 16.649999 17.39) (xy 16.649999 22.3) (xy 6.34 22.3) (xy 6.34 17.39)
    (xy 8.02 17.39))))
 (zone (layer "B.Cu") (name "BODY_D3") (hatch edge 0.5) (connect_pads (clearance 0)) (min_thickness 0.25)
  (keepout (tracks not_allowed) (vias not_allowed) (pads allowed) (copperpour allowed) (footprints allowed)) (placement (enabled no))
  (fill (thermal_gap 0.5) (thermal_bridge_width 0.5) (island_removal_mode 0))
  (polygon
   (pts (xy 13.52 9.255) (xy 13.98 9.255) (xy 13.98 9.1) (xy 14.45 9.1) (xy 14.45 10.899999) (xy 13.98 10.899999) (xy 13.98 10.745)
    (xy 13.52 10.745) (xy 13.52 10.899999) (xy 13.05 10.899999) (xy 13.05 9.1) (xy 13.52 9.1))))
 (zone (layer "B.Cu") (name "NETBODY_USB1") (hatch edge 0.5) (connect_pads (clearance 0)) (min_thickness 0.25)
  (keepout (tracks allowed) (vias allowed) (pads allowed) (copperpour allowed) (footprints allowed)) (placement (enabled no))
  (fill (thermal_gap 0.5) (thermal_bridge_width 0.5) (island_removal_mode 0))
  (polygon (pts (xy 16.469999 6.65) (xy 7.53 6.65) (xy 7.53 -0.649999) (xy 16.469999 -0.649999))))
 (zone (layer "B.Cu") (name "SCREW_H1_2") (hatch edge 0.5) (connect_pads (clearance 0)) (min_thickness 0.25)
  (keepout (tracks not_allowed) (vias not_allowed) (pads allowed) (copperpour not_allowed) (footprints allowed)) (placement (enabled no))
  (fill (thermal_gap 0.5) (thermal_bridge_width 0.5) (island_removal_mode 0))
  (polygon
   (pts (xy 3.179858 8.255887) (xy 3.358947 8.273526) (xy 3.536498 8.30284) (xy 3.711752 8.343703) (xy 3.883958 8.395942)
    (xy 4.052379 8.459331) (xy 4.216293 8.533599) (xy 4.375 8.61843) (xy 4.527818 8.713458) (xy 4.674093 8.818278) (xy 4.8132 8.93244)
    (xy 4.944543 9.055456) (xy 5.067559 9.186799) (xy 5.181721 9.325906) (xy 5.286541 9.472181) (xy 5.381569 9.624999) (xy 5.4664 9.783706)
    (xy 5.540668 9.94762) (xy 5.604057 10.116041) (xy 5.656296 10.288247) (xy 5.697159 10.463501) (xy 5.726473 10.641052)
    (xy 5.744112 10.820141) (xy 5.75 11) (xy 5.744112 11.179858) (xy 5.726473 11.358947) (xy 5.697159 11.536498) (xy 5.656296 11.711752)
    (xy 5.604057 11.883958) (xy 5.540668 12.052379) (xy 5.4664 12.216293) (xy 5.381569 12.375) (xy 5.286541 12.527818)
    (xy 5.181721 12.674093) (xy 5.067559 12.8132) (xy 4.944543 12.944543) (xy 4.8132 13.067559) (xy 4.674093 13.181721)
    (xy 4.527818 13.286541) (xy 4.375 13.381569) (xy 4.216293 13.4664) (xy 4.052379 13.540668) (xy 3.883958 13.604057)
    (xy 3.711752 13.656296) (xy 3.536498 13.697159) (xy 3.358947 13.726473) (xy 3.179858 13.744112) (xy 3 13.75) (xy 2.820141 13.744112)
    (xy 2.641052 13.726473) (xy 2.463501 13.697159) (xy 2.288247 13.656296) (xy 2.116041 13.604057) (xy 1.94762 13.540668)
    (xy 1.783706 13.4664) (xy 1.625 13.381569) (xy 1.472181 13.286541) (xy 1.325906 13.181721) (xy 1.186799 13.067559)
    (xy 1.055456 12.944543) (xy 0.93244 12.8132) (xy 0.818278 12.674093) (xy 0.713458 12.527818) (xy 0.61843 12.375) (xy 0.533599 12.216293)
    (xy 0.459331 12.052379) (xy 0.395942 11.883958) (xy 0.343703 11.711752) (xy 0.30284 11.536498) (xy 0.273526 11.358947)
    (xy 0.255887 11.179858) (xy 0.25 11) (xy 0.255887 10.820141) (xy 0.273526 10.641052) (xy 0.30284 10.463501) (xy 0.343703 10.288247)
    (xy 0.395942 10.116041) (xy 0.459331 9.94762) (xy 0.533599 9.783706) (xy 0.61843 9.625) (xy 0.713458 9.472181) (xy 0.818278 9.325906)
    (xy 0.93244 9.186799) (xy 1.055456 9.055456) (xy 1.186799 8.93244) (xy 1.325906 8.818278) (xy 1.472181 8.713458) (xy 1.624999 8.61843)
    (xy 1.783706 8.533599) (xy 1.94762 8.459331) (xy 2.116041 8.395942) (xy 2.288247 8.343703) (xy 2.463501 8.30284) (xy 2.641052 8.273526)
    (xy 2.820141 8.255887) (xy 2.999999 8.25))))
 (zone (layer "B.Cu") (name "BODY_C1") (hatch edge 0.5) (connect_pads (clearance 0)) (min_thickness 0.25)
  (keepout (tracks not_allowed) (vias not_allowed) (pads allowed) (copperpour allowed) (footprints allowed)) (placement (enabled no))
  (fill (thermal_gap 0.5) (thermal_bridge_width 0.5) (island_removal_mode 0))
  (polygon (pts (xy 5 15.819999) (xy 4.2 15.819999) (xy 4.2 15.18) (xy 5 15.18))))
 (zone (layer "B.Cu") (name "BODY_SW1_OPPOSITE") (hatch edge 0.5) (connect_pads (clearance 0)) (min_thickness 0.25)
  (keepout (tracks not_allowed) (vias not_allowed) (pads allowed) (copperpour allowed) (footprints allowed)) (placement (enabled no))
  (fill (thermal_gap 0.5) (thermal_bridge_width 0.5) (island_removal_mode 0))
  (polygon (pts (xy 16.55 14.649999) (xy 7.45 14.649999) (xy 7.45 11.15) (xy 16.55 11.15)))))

